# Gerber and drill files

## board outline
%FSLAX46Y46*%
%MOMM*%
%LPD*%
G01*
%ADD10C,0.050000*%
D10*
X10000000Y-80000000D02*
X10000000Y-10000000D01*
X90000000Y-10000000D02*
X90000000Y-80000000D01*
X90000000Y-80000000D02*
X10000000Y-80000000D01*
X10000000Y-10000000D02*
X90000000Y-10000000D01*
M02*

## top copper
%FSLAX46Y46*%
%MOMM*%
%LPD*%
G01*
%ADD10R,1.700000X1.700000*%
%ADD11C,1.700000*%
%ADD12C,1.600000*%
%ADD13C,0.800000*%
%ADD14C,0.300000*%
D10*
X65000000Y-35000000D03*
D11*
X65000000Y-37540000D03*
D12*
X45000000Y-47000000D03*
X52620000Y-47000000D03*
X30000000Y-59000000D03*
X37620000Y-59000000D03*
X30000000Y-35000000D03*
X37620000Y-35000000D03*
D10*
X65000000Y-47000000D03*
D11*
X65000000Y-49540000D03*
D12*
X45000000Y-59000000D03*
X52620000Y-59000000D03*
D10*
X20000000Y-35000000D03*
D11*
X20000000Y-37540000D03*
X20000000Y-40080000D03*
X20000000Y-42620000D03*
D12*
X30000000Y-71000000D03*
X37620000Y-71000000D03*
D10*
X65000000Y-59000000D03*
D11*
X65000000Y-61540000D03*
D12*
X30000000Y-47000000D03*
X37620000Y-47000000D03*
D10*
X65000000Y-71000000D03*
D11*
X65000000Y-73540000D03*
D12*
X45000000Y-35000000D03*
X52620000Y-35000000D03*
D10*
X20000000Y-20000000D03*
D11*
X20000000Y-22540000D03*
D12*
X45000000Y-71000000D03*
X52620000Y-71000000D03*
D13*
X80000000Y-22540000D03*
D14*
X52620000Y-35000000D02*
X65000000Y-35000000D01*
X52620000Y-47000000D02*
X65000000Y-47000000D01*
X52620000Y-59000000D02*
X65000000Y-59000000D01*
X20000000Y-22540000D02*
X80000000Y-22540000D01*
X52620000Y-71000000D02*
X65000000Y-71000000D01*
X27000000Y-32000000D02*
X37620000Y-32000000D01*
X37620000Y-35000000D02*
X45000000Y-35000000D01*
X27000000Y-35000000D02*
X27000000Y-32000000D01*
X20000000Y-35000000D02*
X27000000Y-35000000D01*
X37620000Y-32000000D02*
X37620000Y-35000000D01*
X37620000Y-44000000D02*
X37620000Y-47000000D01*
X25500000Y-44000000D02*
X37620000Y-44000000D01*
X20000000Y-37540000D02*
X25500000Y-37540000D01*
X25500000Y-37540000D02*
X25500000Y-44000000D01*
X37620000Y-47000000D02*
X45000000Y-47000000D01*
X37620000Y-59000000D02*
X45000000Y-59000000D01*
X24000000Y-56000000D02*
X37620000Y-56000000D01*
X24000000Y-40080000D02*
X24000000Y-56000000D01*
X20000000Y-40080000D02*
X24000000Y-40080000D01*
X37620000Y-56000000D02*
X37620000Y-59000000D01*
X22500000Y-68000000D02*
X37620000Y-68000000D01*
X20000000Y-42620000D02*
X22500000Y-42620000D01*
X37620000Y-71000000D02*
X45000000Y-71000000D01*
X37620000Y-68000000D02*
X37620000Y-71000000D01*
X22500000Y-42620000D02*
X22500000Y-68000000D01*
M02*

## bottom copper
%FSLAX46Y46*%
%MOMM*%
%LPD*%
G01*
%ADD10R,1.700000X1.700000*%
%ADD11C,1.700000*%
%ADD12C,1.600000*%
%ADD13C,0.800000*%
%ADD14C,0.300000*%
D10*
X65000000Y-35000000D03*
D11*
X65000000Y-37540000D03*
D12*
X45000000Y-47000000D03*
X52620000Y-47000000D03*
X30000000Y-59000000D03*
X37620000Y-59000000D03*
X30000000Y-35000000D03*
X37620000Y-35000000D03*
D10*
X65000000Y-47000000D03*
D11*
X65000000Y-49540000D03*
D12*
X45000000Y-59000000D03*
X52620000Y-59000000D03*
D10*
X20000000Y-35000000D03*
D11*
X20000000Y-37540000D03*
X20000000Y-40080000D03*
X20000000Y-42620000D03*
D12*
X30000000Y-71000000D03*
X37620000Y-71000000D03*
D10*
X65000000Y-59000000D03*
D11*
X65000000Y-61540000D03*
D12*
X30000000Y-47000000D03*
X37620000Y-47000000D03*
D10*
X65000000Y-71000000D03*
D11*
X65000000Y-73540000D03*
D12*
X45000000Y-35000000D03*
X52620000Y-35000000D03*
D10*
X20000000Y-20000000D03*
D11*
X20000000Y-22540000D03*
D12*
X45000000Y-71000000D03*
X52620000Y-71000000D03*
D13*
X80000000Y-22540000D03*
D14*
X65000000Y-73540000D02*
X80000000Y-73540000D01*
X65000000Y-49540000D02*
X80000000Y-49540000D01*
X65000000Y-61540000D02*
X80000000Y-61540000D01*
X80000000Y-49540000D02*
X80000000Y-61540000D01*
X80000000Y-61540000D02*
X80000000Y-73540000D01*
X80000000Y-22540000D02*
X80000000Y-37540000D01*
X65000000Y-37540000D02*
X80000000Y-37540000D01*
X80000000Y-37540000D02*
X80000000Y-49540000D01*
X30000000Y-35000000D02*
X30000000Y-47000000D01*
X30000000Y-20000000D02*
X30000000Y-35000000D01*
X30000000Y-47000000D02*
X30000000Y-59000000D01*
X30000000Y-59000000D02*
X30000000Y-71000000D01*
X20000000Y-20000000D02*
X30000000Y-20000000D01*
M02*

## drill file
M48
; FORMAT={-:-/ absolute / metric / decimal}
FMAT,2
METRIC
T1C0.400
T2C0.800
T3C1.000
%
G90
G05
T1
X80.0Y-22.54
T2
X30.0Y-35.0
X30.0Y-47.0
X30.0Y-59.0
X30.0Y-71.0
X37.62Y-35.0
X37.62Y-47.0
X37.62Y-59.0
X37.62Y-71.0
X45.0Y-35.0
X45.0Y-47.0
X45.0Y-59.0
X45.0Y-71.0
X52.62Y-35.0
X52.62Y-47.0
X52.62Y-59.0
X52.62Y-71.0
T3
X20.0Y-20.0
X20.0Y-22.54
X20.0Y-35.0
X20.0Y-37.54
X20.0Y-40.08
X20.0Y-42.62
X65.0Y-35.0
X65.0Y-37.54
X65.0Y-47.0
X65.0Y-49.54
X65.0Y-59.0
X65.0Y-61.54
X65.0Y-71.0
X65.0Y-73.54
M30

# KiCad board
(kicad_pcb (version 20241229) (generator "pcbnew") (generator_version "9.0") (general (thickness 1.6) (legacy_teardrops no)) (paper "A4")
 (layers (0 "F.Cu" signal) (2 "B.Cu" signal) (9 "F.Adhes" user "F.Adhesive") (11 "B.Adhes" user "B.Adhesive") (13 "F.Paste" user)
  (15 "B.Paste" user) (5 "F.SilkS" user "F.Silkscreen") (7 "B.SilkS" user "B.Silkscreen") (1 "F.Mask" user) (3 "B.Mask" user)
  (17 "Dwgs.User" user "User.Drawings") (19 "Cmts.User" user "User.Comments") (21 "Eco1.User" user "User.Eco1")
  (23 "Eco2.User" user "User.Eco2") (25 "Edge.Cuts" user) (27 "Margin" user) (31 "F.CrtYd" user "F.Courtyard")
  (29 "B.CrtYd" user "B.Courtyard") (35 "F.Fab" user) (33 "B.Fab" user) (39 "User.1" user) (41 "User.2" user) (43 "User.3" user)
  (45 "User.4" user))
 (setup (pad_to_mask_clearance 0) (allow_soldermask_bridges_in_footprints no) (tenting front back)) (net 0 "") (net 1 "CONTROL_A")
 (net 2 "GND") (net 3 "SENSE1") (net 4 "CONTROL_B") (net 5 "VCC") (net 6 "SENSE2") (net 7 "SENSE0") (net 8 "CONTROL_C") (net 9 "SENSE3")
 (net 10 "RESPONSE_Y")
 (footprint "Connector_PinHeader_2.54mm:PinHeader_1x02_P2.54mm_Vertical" (layer "F.Cu") (at 65 35)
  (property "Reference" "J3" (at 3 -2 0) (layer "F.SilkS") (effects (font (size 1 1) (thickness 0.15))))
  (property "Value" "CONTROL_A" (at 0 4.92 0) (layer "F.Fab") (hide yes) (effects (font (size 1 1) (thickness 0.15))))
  (pad "1" thru_hole rect (at 0 0) (size 1.7 1.7) (drill 1) (layers "*.Cu" "*.Mask") (remove_unused_layers no) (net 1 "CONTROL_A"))
  (pad "2" thru_hole circle (at 0 2.54) (size 1.7 1.7) (drill 1) (layers "*.Cu" "*.Mask") (remove_unused_layers no) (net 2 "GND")))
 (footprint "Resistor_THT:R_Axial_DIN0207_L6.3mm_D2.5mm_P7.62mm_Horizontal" (layer "F.Cu") (at 45 47)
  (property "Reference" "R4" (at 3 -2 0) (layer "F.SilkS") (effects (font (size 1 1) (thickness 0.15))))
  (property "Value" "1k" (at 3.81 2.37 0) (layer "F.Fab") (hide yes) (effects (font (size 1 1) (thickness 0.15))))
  (pad "1" thru_hole circle (at 0 0) (size 1.6 1.6) (drill 0.8) (layers "*.Cu" "*.Mask") (remove_unused_layers no) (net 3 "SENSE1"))
  (pad "2" thru_hole circle (at 7.62 0) (size 1.6 1.6) (drill 0.8) (layers "*.Cu" "*.Mask") (remove_unused_layers no) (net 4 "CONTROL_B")))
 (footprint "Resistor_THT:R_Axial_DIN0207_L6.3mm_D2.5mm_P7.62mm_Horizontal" (layer "F.Cu") (at 30 59)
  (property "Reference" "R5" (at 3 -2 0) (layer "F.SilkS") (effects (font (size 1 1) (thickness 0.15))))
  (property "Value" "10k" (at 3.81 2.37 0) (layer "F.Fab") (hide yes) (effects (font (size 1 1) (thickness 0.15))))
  (pad "1" thru_hole circle (at 0 0) (size 1.6 1.6) (drill 0.8) (layers "*.Cu" "*.Mask") (remove_unused_layers no) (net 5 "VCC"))
  (pad "2" thru_hole circle (at 7.62 0) (size 1.6 1.6) (drill 0.8) (layers "*.Cu" "*.Mask") (remove_unused_layers no) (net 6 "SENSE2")))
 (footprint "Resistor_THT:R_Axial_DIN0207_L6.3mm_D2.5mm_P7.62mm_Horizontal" (layer "F.Cu") (at 30 35)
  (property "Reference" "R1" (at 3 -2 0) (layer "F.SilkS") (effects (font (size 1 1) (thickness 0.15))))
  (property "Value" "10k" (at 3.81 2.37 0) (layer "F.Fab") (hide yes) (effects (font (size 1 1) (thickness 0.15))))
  (pad "1" thru_hole circle (at 0 0) (size 1.6 1.6) (drill 0.8) (layers "*.Cu" "*.Mask") (remove_unused_layers no) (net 5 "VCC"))
  (pad "2" thru_hole circle (at 7.62 0) (size 1.6 1.6) (drill 0.8) (layers "*.Cu" "*.Mask") (remove_unused_layers no) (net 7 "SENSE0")))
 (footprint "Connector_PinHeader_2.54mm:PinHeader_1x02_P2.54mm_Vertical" (layer "F.Cu") (at 65 47)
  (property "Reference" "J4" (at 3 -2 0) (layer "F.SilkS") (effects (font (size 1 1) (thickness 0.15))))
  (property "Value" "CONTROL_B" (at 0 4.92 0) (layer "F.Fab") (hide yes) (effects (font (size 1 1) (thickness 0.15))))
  (pad "1" thru_hole rect (at 0 0) (size 1.7 1.7) (drill 1) (layers "*.Cu" "*.Mask") (remove_unused_layers no) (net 4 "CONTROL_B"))
  (pad "2" thru_hole circle (at 0 2.54) (size 1.7 1.7) (drill 1) (layers "*.Cu" "*.Mask") (remove_unused_layers no) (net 2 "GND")))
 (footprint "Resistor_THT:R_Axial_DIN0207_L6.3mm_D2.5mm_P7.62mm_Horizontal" (layer "F.Cu") (at 45 59)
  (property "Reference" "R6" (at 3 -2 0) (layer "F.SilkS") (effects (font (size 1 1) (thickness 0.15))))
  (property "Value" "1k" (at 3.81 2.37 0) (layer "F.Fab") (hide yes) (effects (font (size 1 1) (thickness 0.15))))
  (pad "1" thru_hole circle (at 0 0) (size 1.6 1.6) (drill 0.8) (layers "*.Cu" "*.Mask") (remove_unused_layers no) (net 6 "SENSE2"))
  (pad "2" thru_hole circle (at 7.62 0) (size 1.6 1.6) (drill 0.8) (layers "*.Cu" "*.Mask") (remove_unused_layers no) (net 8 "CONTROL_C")))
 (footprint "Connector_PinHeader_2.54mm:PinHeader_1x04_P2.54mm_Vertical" (layer "F.Cu") (at 20 35)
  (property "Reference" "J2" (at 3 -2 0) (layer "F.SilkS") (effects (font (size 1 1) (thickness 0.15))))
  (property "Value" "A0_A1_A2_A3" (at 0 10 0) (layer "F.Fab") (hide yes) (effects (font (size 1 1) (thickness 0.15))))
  (pad "1" thru_hole rect (at 0 0) (size 1.7 1.7) (drill 1) (layers "*.Cu" "*.Mask") (remove_unused_layers no) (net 7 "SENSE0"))
  (pad "2" thru_hole circle (at 0 2.54) (size 1.7 1.7) (drill 1) (layers "*.Cu" "*.Mask") (remove_unused_layers no) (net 3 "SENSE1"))
  (pad "3" thru_hole circle (at 0 5.08) (size 1.7 1.7) (drill 1) (layers "*.Cu" "*.Mask") (remove_unused_layers no) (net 6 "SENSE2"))
  (pad "4" thru_hole circle (at 0 7.62) (size 1.7 1.7) (drill 1) (layers "*.Cu" "*.Mask") (remove_unused_layers no) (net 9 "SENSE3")))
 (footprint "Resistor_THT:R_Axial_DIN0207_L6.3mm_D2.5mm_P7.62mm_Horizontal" (layer "F.Cu") (at 30 71)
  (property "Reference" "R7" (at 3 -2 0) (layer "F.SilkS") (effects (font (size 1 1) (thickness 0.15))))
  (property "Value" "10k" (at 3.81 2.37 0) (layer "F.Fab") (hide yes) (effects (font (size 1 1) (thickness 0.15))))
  (pad "1" thru_hole circle (at 0 0) (size 1.6 1.6) (drill 0.8) (layers "*.Cu" "*.Mask") (remove_unused_layers no) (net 5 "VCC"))
  (pad "2" thru_hole circle (at 7.62 0) (size 1.6 1.6) (drill 0.8) (layers "*.Cu" "*.Mask") (remove_unused_layers no) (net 9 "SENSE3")))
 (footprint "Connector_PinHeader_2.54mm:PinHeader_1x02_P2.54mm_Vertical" (layer "F.Cu") (at 65 59)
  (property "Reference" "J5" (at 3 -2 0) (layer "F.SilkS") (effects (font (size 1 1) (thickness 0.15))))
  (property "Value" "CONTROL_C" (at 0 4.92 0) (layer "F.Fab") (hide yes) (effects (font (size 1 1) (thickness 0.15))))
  (pad "1" thru_hole rect (at 0 0) (size 1.7 1.7) (drill 1) (layers "*.Cu" "*.Mask") (remove_unused_layers no) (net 8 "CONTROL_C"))
  (pad "2" thru_hole circle (at 0 2.54) (size 1.7 1.7) (drill 1) (layers "*.Cu" "*.Mask") (remove_unused_layers no) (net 2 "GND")))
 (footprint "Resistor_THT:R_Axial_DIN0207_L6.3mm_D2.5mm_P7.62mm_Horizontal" (layer "F.Cu") (at 30 47)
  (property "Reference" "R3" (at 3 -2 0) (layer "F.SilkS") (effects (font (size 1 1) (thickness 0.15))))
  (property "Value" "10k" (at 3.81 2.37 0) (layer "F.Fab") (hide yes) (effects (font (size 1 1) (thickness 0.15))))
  (pad "1" thru_hole circle (at 0 0) (size 1.6 1.6) (drill 0.8) (layers "*.Cu" "*.Mask") (remove_unused_layers no) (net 5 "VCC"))
  (pad "2" thru_hole circle (at 7.62 0) (size 1.6 1.6) (drill 0.8) (layers "*.Cu" "*.Mask") (remove_unused_layers no) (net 3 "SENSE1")))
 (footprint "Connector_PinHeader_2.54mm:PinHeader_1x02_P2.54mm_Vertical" (layer "F.Cu") (at 65 71)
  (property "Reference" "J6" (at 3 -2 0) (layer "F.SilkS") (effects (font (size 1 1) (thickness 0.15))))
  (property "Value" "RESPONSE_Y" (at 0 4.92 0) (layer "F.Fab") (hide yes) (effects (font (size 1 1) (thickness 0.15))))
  (pad "1" thru_hole rect (at 0 0) (size 1.7 1.7) (drill 1) (layers "*.Cu" "*.Mask") (remove_unused_layers no) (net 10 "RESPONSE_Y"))
  (pad "2" thru_hole circle (at 0 2.54) (size 1.7 1.7) (drill 1) (layers "*.Cu" "*.Mask") (remove_unused_layers no) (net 2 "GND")))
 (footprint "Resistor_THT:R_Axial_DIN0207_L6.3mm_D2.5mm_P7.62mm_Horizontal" (layer "F.Cu") (at 45 35)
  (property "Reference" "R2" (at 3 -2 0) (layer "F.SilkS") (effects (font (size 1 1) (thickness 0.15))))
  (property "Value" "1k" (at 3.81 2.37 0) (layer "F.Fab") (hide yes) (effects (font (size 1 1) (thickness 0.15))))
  (pad "1" thru_hole circle (at 0 0) (size 1.6 1.6) (drill 0.8) (layers "*.Cu" "*.Mask") (remove_unused_layers no) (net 7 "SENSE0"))
  (pad "2" thru_hole circle (at 7.62 0) (size 1.6 1.6) (drill 0.8) (layers "*.Cu" "*.Mask") (remove_unused_layers no) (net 1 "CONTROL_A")))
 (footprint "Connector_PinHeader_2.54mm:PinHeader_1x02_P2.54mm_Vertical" (layer "F.Cu") (at 20 20)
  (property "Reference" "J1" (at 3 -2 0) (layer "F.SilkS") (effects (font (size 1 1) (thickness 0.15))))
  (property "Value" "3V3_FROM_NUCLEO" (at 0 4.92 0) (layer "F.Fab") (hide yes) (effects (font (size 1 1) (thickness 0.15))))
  (pad "1" thru_hole rect (at 0 0) (size 1.7 1.7) (drill 1) (layers "*.Cu" "*.Mask") (remove_unused_layers no) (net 5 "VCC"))
  (pad "2" thru_hole circle (at 0 2.54) (size 1.7 1.7) (drill 1) (layers "*.Cu" "*.Mask") (remove_unused_layers no) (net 2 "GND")))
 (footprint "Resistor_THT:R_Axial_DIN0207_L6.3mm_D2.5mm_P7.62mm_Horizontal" (layer "F.Cu") (at 45 71)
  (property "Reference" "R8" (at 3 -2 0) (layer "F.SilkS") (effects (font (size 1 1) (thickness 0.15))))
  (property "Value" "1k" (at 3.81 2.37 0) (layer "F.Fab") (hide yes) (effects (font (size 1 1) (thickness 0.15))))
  (pad "1" thru_hole circle (at 0 0) (size 1.6 1.6) (drill 0.8) (layers "*.Cu" "*.Mask") (remove_unused_layers no) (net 9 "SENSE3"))
  (pad "2" thru_hole circle (at 7.62 0) (size 1.6 1.6) (drill 0.8) (layers "*.Cu" "*.Mask") (remove_unused_layers no) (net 10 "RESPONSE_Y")))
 (gr_line (start 10 80) (end 10 10) (stroke (width 0.05) (type default)) (layer "Edge.Cuts"))
 (gr_line (start 90 10) (end 90 80) (stroke (width 0.05) (type default)) (layer "Edge.Cuts"))
 (gr_line (start 90 80) (end 10 80) (stroke (width 0.05) (type default)) (layer "Edge.Cuts"))
 (gr_line (start 10 10) (end 90 10) (stroke (width 0.05) (type default)) (layer "Edge.Cuts"))
 (segment (start 52.62 35) (end 65 35) (width 0.3) (layer "F.Cu") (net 1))
 (segment (start 52.62 47) (end 65 47) (width 0.3) (layer "F.Cu") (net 4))
 (segment (start 52.62 59) (end 65 59) (width 0.3) (layer "F.Cu") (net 8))
 (segment (start 20 22.54) (end 80 22.54) (width 0.3) (layer "F.Cu") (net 2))
 (via (at 80 22.54) (size 0.8) (drill 0.4) (layers "F.Cu" "B.Cu") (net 2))
 (segment (start 65 73.54) (end 80 73.54) (width 0.3) (layer "B.Cu") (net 2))
 (segment (start 65 49.54) (end 80 49.54) (width 0.3) (layer "B.Cu") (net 2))
 (segment (start 65 61.54) (end 80 61.54) (width 0.3) (layer "B.Cu") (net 2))
 (segment (start 80 49.54) (end 80 61.54) (width 0.3) (layer "B.Cu") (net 2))
 (segment (start 80 61.54) (end 80 73.54) (width 0.3) (layer "B.Cu") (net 2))
 (segment (start 80 22.54) (end 80 37.54) (width 0.3) (layer "B.Cu") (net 2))
 (segment (start 65 37.54) (end 80 37.54) (width 0.3) (layer "B.Cu") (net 2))
 (segment (start 80 37.54) (end 80 49.54) (width 0.3) (layer "B.Cu") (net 2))
 (segment (start 52.62 71) (end 65 71) (width 0.3) (layer "F.Cu") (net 10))
 (segment (start 27 32) (end 37.62 32) (width 0.3) (layer "F.Cu") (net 7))
 (segment (start 37.62 35) (end 45 35) (width 0.3) (layer "F.Cu") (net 7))
 (segment (start 27 35) (end 27 32) (width 0.3) (layer "F.Cu") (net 7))
 (segment (start 20 35) (end 27 35) (width 0.3) (layer "F.Cu") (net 7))
 (segment (start 37.62 32) (end 37.62 35) (width 0.3) (layer "F.Cu") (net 7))
 (segment (start 37.62 44) (end 37.62 47) (width 0.3) (layer "F.Cu") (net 3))
 (segment (start 25.5 44) (end 37.62 44) (width 0.3) (layer "F.Cu") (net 3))
 (segment (start 20 37.54) (end 25.5 37.54) (width 0.3) (layer "F.Cu") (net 3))
 (segment (start 25.5 37.54) (end 25.5 44) (width 0.3) (layer "F.Cu") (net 3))
 (segment (start 37.62 47) (end 45 47) (width 0.3) (layer "F.Cu") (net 3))
 (segment (start 37.62 59) (end 45 59) (width 0.3) (layer "F.Cu") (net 6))
 (segment (start 24 56) (end 37.62 56) (width 0.3) (layer "F.Cu") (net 6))
 (segment (start 24 40.08) (end 24 56) (width 0.3) (layer "F.Cu") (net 6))
 (segment (start 20 40.08) (end 24 40.08) (width 0.3) (layer "F.Cu") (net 6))
 (segment (start 37.62 56) (end 37.62 59) (width 0.3) (layer "F.Cu") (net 6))
 (segment (start 22.5 68) (end 37.62 68) (width 0.3) (layer "F.Cu") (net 9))
 (segment (start 20 42.62) (end 22.5 42.62) (width 0.3) (layer "F.Cu") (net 9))
 (segment (start 37.62 71) (end 45 71) (width 0.3) (layer "F.Cu") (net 9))
 (segment (start 37.62 68) (end 37.62 71) (width 0.3) (layer "F.Cu") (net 9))
 (segment (start 22.5 42.62) (end 22.5 68) (width 0.3) (layer "F.Cu") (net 9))
 (segment (start 30 35) (end 30 47) (width 0.3) (layer "B.Cu") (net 5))
 (segment (start 30 20) (end 30 35) (width 0.3) (layer "B.Cu") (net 5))
 (segment (start 30 47) (end 30 59) (width 0.3) (layer "B.Cu") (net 5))
 (segment (start 30 59) (end 30 71) (width 0.3) (layer "B.Cu") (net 5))
 (segment (start 20 20) (end 30 20) (width 0.3) (layer "B.Cu") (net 5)))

